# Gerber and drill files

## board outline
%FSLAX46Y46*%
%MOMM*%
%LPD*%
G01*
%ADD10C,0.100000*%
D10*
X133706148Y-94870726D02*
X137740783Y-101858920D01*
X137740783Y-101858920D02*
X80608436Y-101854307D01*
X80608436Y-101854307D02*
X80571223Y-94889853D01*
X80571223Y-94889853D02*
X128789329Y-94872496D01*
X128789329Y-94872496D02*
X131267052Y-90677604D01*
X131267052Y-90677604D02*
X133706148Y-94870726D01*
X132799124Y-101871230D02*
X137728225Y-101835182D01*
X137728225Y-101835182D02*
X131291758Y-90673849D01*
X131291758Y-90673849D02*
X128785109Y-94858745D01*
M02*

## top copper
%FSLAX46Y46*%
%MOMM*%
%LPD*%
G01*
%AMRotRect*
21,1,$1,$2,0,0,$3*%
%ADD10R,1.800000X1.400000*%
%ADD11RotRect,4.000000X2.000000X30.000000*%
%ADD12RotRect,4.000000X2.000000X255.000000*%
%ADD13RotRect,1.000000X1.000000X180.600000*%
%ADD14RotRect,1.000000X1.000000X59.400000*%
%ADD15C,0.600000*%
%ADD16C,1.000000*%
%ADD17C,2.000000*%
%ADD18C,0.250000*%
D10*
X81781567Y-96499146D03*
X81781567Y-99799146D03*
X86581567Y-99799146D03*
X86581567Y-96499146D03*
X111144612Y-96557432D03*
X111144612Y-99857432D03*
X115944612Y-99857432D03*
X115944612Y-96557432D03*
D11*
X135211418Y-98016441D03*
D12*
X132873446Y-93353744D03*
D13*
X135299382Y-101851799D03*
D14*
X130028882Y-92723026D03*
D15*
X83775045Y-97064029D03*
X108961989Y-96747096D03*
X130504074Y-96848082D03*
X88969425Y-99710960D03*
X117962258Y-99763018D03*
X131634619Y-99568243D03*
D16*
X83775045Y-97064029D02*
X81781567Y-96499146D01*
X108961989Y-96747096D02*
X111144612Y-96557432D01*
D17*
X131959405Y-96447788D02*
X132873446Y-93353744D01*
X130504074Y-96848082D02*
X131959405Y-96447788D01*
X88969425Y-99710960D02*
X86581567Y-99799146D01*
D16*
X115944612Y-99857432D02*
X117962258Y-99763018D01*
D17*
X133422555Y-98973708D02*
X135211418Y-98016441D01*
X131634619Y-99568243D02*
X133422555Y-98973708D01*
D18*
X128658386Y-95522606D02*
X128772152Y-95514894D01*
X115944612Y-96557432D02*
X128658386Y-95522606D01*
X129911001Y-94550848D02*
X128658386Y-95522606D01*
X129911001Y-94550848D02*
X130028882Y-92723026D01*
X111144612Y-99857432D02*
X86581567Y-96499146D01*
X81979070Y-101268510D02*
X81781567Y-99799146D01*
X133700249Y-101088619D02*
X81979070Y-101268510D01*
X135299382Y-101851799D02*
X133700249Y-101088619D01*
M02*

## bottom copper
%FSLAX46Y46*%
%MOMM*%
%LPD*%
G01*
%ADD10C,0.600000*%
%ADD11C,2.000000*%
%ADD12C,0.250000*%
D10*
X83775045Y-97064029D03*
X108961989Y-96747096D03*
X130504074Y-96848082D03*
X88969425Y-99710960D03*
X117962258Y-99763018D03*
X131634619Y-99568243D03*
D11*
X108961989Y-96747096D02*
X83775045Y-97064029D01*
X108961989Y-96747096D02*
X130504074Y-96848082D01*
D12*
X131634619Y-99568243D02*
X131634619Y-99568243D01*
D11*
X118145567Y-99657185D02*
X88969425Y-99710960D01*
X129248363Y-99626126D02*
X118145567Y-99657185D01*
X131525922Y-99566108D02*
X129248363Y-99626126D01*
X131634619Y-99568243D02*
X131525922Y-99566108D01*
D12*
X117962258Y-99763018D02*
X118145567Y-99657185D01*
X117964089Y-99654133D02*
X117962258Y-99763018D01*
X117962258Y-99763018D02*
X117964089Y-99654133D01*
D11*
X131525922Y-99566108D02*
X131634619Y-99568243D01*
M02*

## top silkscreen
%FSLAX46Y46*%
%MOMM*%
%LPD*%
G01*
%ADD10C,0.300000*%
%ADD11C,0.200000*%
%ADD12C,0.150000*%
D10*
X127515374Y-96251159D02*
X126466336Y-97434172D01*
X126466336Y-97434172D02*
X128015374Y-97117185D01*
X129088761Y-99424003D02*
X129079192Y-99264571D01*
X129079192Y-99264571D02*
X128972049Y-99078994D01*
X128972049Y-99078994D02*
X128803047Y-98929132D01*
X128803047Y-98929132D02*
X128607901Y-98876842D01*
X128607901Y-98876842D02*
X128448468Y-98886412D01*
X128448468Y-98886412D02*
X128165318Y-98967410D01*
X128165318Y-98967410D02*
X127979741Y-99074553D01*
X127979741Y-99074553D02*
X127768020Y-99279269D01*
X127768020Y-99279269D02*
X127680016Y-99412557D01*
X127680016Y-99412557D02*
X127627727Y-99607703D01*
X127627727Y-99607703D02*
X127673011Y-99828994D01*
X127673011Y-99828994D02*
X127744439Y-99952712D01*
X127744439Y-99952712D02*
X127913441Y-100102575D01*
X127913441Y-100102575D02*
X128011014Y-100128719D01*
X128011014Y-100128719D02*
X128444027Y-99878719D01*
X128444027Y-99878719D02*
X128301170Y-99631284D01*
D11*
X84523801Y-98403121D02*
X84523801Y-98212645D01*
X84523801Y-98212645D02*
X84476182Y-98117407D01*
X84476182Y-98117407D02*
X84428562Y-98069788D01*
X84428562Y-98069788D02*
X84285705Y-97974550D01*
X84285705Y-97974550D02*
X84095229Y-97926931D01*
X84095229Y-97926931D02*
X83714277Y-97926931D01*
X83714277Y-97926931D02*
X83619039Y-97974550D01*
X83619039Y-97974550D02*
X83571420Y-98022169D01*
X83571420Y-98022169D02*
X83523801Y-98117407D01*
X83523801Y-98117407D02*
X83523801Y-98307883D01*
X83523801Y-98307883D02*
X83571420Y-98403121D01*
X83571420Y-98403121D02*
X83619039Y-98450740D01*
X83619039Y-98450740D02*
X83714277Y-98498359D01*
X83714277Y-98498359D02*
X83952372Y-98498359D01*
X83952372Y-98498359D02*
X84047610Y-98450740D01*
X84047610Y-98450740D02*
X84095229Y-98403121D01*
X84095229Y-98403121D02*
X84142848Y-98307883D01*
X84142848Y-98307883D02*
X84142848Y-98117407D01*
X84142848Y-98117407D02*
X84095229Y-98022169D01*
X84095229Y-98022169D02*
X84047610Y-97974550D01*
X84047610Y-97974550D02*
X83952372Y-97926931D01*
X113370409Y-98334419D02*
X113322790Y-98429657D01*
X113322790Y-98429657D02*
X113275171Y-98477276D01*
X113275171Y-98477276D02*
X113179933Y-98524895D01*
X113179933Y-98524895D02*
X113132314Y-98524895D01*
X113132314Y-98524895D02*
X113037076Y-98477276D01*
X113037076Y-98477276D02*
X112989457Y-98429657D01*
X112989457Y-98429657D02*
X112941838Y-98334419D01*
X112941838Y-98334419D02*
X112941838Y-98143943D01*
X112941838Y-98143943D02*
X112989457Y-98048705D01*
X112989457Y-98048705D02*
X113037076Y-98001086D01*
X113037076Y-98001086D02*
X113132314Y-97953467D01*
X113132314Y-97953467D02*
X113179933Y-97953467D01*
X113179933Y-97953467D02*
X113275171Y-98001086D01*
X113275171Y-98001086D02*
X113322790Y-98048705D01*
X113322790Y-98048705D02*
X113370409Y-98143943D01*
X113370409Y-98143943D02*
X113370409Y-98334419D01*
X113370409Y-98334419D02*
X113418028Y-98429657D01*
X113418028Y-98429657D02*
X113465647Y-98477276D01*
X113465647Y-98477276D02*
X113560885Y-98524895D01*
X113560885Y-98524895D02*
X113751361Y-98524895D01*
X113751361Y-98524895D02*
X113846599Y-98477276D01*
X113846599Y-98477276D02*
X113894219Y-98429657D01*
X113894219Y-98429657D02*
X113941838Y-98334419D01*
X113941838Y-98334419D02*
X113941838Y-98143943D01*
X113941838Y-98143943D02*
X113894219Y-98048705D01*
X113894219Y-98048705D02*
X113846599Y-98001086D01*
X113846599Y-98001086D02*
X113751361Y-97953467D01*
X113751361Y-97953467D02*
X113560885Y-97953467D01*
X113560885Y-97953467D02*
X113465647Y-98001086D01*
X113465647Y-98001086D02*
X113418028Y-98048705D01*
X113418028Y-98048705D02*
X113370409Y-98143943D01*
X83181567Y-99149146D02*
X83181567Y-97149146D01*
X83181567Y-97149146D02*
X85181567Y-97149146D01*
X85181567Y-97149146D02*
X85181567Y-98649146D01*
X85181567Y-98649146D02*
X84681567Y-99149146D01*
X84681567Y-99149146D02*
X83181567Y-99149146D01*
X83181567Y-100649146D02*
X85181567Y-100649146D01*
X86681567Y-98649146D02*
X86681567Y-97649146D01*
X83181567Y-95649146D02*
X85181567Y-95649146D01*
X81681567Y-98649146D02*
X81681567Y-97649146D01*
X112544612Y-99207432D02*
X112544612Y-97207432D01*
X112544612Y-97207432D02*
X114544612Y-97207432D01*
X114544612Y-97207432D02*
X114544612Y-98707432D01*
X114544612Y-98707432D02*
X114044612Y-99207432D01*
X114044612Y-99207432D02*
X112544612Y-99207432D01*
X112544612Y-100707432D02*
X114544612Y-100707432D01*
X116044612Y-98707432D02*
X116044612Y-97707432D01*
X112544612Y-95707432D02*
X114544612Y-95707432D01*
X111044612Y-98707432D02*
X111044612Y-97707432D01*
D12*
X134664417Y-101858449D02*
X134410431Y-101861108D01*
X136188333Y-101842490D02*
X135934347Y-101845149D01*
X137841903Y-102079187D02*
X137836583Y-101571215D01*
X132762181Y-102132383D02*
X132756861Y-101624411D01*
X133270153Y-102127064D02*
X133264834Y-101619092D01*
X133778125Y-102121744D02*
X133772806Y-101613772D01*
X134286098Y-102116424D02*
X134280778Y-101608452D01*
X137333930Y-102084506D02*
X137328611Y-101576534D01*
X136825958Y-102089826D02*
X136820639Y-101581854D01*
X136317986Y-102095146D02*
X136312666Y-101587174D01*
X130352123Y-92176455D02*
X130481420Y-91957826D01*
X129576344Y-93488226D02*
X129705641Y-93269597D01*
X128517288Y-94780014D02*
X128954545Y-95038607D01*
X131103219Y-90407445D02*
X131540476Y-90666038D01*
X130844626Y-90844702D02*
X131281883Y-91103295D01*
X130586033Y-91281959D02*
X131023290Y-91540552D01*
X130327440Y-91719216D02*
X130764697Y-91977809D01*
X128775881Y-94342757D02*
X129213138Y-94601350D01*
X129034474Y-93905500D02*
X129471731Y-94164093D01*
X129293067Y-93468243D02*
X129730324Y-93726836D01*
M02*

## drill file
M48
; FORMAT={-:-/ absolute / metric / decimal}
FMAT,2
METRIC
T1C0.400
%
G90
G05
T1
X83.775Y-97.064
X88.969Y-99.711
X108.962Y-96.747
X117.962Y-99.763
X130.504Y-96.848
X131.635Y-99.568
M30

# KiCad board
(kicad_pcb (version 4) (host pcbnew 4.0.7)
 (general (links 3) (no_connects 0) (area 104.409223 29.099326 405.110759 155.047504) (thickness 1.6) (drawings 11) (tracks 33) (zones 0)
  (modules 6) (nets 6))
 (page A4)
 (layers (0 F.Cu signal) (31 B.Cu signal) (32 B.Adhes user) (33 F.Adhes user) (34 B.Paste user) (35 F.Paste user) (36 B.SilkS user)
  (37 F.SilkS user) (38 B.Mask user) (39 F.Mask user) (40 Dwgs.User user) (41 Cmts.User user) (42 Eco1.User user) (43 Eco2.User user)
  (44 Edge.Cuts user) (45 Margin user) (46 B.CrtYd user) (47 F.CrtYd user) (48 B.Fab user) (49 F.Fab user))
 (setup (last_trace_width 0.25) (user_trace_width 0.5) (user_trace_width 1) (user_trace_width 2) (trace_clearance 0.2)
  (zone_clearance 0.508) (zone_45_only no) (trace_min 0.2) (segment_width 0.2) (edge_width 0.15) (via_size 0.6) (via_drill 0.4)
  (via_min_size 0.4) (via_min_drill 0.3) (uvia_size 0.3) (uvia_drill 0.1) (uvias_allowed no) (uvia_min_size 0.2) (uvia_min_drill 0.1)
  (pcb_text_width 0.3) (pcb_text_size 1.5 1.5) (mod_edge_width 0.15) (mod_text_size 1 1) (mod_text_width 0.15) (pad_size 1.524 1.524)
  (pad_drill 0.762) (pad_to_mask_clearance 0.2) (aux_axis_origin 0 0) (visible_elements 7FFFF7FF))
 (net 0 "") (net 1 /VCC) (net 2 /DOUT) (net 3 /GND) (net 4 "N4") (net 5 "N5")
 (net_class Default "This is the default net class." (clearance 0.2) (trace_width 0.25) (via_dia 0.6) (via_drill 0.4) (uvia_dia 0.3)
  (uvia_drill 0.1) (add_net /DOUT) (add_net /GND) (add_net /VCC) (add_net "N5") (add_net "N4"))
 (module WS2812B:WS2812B (layer F.Cu) (at 84.1815668464366 98.1491456770292 90)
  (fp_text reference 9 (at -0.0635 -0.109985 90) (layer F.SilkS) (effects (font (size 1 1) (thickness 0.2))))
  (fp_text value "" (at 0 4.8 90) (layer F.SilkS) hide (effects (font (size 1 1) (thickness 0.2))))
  (fp_line (start -1 -1) (end 1 -1) (layer F.SilkS) (width 0.2)) (fp_line (start 1 -1) (end 1 1) (layer F.SilkS) (width 0.2))
  (fp_line (start 1 1) (end -0.5 1) (layer F.SilkS) (width 0.2))
  (fp_line (start -0.5 1) (end -1 0.5) (layer F.SilkS) (width 0.2))
  (fp_line (start -1 0.5) (end -1 -1) (layer F.SilkS) (width 0.2))
  (fp_line (start -2.5 -1) (end -2.5 1) (layer F.SilkS) (width 0.2))
  (fp_line (start -0.5 2.5) (end 0.5 2.5) (layer F.SilkS) (width 0.2))
  (fp_line (start 2.5 -1) (end 2.5 1) (layer F.SilkS) (width 0.2))
  (fp_line (start -0.5 -2.5) (end 0.5 -2.5) (layer F.SilkS) (width 0.2))
  (pad 1 smd rect (at 1.65 -2.4 90) (size 1.4 1.8) (layers F.Cu F.Paste F.Mask) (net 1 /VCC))
  (pad 2 smd rect (at -1.65 -2.4 90) (size 1.4 1.8) (layers F.Cu F.Paste F.Mask) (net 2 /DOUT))
  (pad 3 smd rect (at -1.65 2.4 90) (size 1.4 1.8) (layers F.Cu F.Paste F.Mask) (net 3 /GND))
  (pad 4 smd rect (at 1.65 2.4 90) (size 1.4 1.8) (layers F.Cu F.Paste F.Mask) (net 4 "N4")))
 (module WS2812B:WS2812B (layer F.Cu) (at 113.544612102561 98.2074319255815 90)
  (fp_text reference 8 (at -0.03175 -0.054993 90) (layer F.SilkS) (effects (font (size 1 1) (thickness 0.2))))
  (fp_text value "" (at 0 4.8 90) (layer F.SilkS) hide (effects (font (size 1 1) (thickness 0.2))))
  (fp_line (start -1 -1) (end 1 -1) (layer F.SilkS) (width 0.2)) (fp_line (start 1 -1) (end 1 1) (layer F.SilkS) (width 0.2))
  (fp_line (start 1 1) (end -0.5 1) (layer F.SilkS) (width 0.2))
  (fp_line (start -0.5 1) (end -1 0.5) (layer F.SilkS) (width 0.2))
  (fp_line (start -1 0.5) (end -1 -1) (layer F.SilkS) (width 0.2))
  (fp_line (start -2.5 -1) (end -2.5 1) (layer F.SilkS) (width 0.2))
  (fp_line (start -0.5 2.5) (end 0.5 2.5) (layer F.SilkS) (width 0.2))
  (fp_line (start 2.5 -1) (end 2.5 1) (layer F.SilkS) (width 0.2))
  (fp_line (start -0.5 -2.5) (end 0.5 -2.5) (layer F.SilkS) (width 0.2))
  (pad 1 smd rect (at 1.65 -2.4 90) (size 1.4 1.8) (layers F.Cu F.Paste F.Mask) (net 1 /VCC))
  (pad 2 smd rect (at -1.65 -2.4 90) (size 1.4 1.8) (layers F.Cu F.Paste F.Mask) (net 4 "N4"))
  (pad 3 smd rect (at -1.65 2.4 90) (size 1.4 1.8) (layers F.Cu F.Paste F.Mask) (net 3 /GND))
  (pad 4 smd rect (at 1.65 2.4 90) (size 1.4 1.8) (layers F.Cu F.Paste F.Mask) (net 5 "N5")))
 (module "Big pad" (layer F.Cu) (at 135.384903431515 98.0629261594345 30)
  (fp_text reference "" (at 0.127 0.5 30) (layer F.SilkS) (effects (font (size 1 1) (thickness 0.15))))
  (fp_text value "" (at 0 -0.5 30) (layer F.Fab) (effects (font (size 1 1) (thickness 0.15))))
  (pad 1 smd rect (at -0.127 -0.127 30) (size 4 2) (layers F.Cu F.Paste F.Mask)))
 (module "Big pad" (layer F.Cu) (at 132.717903431515 93.4435466556483 255)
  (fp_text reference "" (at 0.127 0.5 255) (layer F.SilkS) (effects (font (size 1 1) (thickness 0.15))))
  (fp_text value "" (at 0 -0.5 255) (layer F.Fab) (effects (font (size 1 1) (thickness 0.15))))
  (pad 1 smd rect (at -0.127 -0.127 255) (size 4 2) (layers F.Cu F.Paste F.Mask)))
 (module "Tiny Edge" (layer F.Cu) (at 135.299382424165 101.85179942959 180.6)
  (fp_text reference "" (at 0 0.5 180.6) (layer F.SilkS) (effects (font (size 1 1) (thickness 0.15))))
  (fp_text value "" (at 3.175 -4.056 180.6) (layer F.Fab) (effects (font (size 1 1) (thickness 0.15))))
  (fp_line (start 0.635 0) (end 0.889 0) (layer F.SilkS) (width 0.15))
  (fp_line (start -0.889 0) (end -0.635 0) (layer F.SilkS) (width 0.15))
  (fp_line (start -2.54 -0.254) (end -2.54 0.254) (layer F.SilkS) (width 0.15))
  (fp_line (start 2.54 -0.254) (end 2.54 0.254) (layer F.SilkS) (width 0.15))
  (fp_line (start 2.032 -0.254) (end 2.032 0.254) (layer F.SilkS) (width 0.15))
  (fp_line (start 1.524 -0.254) (end 1.524 0.254) (layer F.SilkS) (width 0.15))
  (fp_line (start 1.016 -0.254) (end 1.016 0.254) (layer F.SilkS) (width 0.15))
  (fp_line (start -2.032 -0.254) (end -2.032 0.254) (layer F.SilkS) (width 0.15))
  (fp_line (start -1.524 -0.254) (end -1.524 0.254) (layer F.SilkS) (width 0.15))
  (fp_line (start -1.016 -0.254) (end -1.016 0.254) (layer F.SilkS) (width 0.15))
  (pad 1 smd rect (at 0 0 180.6) (size 1 1) (layers F.Cu F.Paste F.Mask)))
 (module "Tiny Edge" (layer F.Cu) (at 130.028882424165 92.7230256482987 59.4)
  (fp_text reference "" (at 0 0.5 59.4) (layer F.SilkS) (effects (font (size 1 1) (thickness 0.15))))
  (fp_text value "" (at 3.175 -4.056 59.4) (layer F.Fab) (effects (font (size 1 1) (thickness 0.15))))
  (fp_line (start 0.635 0) (end 0.889 0) (layer F.SilkS) (width 0.15))
  (fp_line (start -0.889 0) (end -0.635 0) (layer F.SilkS) (width 0.15))
  (fp_line (start -2.54 -0.254) (end -2.54 0.254) (layer F.SilkS) (width 0.15))
  (fp_line (start 2.54 -0.254) (end 2.54 0.254) (layer F.SilkS) (width 0.15))
  (fp_line (start 2.032 -0.254) (end 2.032 0.254) (layer F.SilkS) (width 0.15))
  (fp_line (start 1.524 -0.254) (end 1.524 0.254) (layer F.SilkS) (width 0.15))
  (fp_line (start 1.016 -0.254) (end 1.016 0.254) (layer F.SilkS) (width 0.15))
  (fp_line (start -2.032 -0.254) (end -2.032 0.254) (layer F.SilkS) (width 0.15))
  (fp_line (start -1.524 -0.254) (end -1.524 0.254) (layer F.SilkS) (width 0.15))
  (fp_line (start -1.016 -0.254) (end -1.016 0.254) (layer F.SilkS) (width 0.15))
  (pad 1 smd rect (at 0 0 59.4) (size 1 1) (layers F.Cu F.Paste F.Mask)))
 (gr_line (start 133.70614787533 94.8707262426342) (end 137.74078337533 101.858919918655) (layer Edge.Cuts) (width 0.1))
 (gr_line (start 137.74078337533 101.858919918655) (end 80.6084355758387 101.854306774241) (layer Edge.Cuts) (width 0.1))
 (gr_line (start 80.6084355758387 101.854306774241) (end 80.5712232188951 94.8898530813448) (layer Edge.Cuts) (width 0.1))
 (gr_line (start 80.5712232188951 94.8898530813448) (end 128.789328831247 94.8724958466605) (layer Edge.Cuts) (width 0.1))
 (gr_line (start 128.789328831247 94.8724958466605) (end 131.267052047017 90.6776043434671) (layer Edge.Cuts) (width 0.1))
 (gr_line (start 131.267052047017 90.6776043434671) (end 133.70614787533 94.8707262426342) (layer Edge.Cuts) (width 0.1))
 (gr_line (start 132.799123572858 101.871230067052) (end 137.728224838556 101.835181894894) (layer Edge.Cuts) (width 0.1))
 (gr_line (start 137.728224838556 101.835181894894) (end 131.291758422265 90.6738490406669) (layer Edge.Cuts) (width 0.1))
 (gr_line (start 131.291758422265 90.6738490406669) (end 128.785108799073 94.8587445365249) (layer Edge.Cuts) (width 0.1))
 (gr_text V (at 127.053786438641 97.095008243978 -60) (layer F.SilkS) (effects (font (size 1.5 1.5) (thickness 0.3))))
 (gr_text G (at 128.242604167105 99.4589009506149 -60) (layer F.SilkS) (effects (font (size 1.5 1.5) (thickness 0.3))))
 (segment (start 108.961988832405 96.7470955897241) (end 83.7750446858575 97.0640286405036) (width 2) (layer B.Cu) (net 1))
 (via (at 83.7750446858575 97.0640286405036) (size 0.6) (drill 0.4) (layers F.Cu B.Cu) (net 1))
 (segment (start 83.7750446858575 97.0640286405036) (end 81.7815667777835 96.4991456199533) (width 1) (layer F.Cu) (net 1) (status 20))
 (segment (start 108.961988832405 96.7470955897241) (end 111.144612033908 96.5574318685057) (width 1) (layer F.Cu) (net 1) (status 20))
 (via (at 108.961988832405 96.7470955897241) (size 0.6) (drill 0.4) (layers F.Cu B.Cu) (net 1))
 (segment (start 108.961988832405 96.7470955897241) (end 130.504074482517 96.8480824367174) (width 2) (layer B.Cu) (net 1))
 (segment (start 131.959404584744 96.4477881155593) (end 132.873445924161 93.3537441556483) (width 2) (layer F.Cu) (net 1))
 (segment (start 130.504074482517 96.8480824367174) (end 131.959404584744 96.4477881155593) (width 2) (layer F.Cu) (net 1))
 (via (at 130.504074482517 96.8480824367174) (size 0.6) (drill 0.4) (layers F.Cu B.Cu) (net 1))
 (segment (start 131.634618803675 99.5682426411717) (end 131.634618803675 99.5682426411717) (width 0.25) (layer B.Cu) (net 3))
 (via (at 88.9694253428731 99.7109598523076) (size 0.6) (drill 0.4) (layers F.Cu B.Cu) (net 3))
 (segment (start 88.9694253428731 99.7109598523076) (end 86.5815669150896 99.7991457341051) (width 2) (layer F.Cu) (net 3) (status 20))
 (segment (start 118.145566532439 99.657184761439) (end 88.9694253428731 99.7109598523076) (width 2) (layer B.Cu) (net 3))
 (segment (start 129.248362570045 99.6261256046461) (end 118.145566532439 99.657184761439) (width 2) (layer B.Cu) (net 3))
 (segment (start 131.525921917421 99.5661081115553) (end 129.248362570045 99.6261256046461) (width 2) (layer B.Cu) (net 3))
 (segment (start 131.634618803675 99.5682426411717) (end 131.525921917421 99.5661081115553) (width 2) (layer B.Cu) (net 3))
 (segment (start 117.962257533296 99.763018261439) (end 118.145566532439 99.657184761439) (width 0.25) (layer B.Cu) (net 3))
 (segment (start 117.964089070645 99.6541325771828) (end 117.962257533296 99.763018261439) (width 0.25) (layer B.Cu) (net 3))
 (segment (start 117.962257533296 99.763018261439) (end 117.964089070645 99.6541325771828) (width 0.25) (layer B.Cu) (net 3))
 (via (at 117.962257533296 99.763018261439) (size 0.6) (drill 0.4) (layers F.Cu B.Cu) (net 3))
 (segment (start 115.944612171214 99.8574319826574) (end 117.962257533296 99.763018261439) (width 1) (layer F.Cu) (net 3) (status 10))
 (segment (start 133.422555446576 98.9737077473908) (end 135.211418205234 98.0164409331539) (width 2) (layer F.Cu) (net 3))
 (segment (start 131.634618803675 99.5682426411717) (end 133.422555446576 98.9737077473908) (width 2) (layer F.Cu) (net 3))
 (via (at 131.634618803675 99.5682426411717) (size 0.6) (drill 0.4) (layers F.Cu B.Cu) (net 3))
 (segment (start 131.525921917421 99.5661081115553) (end 131.634618803675 99.5682426411717) (width 2) (layer B.Cu) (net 3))
 (segment (start 128.658385662831 95.5226056260594) (end 128.77215184367 95.5148944314564) (width 0.25) (layer F.Cu) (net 5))
 (segment (start 115.944612087459 96.5574318375883) (end 128.658385662831 95.5226056260594) (width 0.25) (layer F.Cu) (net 5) (status 10))
 (segment (start 129.91100061392 94.5508483636662) (end 128.658385662831 95.5226056260594) (width 0.25) (layer F.Cu) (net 5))
 (segment (start 129.91100061392 94.5508483636662) (end 130.028882424165 92.7230256482987) (width 0.25) (layer F.Cu) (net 5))
 (segment (start 111.144612117664 99.8574320135748) (end 86.5815668313339 96.499145589036) (width 0.25) (layer F.Cu) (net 4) (status 20))
 (segment (start 81.9790701689756 101.268509528165) (end 81.7815668615392 99.7991457650224) (width 0.25) (layer F.Cu) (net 2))
 (segment (start 133.700249136548 101.088619327363) (end 81.9790701689756 101.268509528165) (width 0.25) (layer F.Cu) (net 2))
 (segment (start 135.299382424165 101.85179942959) (end 133.700249136548 101.088619327363) (width 0.25) (layer F.Cu) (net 2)))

